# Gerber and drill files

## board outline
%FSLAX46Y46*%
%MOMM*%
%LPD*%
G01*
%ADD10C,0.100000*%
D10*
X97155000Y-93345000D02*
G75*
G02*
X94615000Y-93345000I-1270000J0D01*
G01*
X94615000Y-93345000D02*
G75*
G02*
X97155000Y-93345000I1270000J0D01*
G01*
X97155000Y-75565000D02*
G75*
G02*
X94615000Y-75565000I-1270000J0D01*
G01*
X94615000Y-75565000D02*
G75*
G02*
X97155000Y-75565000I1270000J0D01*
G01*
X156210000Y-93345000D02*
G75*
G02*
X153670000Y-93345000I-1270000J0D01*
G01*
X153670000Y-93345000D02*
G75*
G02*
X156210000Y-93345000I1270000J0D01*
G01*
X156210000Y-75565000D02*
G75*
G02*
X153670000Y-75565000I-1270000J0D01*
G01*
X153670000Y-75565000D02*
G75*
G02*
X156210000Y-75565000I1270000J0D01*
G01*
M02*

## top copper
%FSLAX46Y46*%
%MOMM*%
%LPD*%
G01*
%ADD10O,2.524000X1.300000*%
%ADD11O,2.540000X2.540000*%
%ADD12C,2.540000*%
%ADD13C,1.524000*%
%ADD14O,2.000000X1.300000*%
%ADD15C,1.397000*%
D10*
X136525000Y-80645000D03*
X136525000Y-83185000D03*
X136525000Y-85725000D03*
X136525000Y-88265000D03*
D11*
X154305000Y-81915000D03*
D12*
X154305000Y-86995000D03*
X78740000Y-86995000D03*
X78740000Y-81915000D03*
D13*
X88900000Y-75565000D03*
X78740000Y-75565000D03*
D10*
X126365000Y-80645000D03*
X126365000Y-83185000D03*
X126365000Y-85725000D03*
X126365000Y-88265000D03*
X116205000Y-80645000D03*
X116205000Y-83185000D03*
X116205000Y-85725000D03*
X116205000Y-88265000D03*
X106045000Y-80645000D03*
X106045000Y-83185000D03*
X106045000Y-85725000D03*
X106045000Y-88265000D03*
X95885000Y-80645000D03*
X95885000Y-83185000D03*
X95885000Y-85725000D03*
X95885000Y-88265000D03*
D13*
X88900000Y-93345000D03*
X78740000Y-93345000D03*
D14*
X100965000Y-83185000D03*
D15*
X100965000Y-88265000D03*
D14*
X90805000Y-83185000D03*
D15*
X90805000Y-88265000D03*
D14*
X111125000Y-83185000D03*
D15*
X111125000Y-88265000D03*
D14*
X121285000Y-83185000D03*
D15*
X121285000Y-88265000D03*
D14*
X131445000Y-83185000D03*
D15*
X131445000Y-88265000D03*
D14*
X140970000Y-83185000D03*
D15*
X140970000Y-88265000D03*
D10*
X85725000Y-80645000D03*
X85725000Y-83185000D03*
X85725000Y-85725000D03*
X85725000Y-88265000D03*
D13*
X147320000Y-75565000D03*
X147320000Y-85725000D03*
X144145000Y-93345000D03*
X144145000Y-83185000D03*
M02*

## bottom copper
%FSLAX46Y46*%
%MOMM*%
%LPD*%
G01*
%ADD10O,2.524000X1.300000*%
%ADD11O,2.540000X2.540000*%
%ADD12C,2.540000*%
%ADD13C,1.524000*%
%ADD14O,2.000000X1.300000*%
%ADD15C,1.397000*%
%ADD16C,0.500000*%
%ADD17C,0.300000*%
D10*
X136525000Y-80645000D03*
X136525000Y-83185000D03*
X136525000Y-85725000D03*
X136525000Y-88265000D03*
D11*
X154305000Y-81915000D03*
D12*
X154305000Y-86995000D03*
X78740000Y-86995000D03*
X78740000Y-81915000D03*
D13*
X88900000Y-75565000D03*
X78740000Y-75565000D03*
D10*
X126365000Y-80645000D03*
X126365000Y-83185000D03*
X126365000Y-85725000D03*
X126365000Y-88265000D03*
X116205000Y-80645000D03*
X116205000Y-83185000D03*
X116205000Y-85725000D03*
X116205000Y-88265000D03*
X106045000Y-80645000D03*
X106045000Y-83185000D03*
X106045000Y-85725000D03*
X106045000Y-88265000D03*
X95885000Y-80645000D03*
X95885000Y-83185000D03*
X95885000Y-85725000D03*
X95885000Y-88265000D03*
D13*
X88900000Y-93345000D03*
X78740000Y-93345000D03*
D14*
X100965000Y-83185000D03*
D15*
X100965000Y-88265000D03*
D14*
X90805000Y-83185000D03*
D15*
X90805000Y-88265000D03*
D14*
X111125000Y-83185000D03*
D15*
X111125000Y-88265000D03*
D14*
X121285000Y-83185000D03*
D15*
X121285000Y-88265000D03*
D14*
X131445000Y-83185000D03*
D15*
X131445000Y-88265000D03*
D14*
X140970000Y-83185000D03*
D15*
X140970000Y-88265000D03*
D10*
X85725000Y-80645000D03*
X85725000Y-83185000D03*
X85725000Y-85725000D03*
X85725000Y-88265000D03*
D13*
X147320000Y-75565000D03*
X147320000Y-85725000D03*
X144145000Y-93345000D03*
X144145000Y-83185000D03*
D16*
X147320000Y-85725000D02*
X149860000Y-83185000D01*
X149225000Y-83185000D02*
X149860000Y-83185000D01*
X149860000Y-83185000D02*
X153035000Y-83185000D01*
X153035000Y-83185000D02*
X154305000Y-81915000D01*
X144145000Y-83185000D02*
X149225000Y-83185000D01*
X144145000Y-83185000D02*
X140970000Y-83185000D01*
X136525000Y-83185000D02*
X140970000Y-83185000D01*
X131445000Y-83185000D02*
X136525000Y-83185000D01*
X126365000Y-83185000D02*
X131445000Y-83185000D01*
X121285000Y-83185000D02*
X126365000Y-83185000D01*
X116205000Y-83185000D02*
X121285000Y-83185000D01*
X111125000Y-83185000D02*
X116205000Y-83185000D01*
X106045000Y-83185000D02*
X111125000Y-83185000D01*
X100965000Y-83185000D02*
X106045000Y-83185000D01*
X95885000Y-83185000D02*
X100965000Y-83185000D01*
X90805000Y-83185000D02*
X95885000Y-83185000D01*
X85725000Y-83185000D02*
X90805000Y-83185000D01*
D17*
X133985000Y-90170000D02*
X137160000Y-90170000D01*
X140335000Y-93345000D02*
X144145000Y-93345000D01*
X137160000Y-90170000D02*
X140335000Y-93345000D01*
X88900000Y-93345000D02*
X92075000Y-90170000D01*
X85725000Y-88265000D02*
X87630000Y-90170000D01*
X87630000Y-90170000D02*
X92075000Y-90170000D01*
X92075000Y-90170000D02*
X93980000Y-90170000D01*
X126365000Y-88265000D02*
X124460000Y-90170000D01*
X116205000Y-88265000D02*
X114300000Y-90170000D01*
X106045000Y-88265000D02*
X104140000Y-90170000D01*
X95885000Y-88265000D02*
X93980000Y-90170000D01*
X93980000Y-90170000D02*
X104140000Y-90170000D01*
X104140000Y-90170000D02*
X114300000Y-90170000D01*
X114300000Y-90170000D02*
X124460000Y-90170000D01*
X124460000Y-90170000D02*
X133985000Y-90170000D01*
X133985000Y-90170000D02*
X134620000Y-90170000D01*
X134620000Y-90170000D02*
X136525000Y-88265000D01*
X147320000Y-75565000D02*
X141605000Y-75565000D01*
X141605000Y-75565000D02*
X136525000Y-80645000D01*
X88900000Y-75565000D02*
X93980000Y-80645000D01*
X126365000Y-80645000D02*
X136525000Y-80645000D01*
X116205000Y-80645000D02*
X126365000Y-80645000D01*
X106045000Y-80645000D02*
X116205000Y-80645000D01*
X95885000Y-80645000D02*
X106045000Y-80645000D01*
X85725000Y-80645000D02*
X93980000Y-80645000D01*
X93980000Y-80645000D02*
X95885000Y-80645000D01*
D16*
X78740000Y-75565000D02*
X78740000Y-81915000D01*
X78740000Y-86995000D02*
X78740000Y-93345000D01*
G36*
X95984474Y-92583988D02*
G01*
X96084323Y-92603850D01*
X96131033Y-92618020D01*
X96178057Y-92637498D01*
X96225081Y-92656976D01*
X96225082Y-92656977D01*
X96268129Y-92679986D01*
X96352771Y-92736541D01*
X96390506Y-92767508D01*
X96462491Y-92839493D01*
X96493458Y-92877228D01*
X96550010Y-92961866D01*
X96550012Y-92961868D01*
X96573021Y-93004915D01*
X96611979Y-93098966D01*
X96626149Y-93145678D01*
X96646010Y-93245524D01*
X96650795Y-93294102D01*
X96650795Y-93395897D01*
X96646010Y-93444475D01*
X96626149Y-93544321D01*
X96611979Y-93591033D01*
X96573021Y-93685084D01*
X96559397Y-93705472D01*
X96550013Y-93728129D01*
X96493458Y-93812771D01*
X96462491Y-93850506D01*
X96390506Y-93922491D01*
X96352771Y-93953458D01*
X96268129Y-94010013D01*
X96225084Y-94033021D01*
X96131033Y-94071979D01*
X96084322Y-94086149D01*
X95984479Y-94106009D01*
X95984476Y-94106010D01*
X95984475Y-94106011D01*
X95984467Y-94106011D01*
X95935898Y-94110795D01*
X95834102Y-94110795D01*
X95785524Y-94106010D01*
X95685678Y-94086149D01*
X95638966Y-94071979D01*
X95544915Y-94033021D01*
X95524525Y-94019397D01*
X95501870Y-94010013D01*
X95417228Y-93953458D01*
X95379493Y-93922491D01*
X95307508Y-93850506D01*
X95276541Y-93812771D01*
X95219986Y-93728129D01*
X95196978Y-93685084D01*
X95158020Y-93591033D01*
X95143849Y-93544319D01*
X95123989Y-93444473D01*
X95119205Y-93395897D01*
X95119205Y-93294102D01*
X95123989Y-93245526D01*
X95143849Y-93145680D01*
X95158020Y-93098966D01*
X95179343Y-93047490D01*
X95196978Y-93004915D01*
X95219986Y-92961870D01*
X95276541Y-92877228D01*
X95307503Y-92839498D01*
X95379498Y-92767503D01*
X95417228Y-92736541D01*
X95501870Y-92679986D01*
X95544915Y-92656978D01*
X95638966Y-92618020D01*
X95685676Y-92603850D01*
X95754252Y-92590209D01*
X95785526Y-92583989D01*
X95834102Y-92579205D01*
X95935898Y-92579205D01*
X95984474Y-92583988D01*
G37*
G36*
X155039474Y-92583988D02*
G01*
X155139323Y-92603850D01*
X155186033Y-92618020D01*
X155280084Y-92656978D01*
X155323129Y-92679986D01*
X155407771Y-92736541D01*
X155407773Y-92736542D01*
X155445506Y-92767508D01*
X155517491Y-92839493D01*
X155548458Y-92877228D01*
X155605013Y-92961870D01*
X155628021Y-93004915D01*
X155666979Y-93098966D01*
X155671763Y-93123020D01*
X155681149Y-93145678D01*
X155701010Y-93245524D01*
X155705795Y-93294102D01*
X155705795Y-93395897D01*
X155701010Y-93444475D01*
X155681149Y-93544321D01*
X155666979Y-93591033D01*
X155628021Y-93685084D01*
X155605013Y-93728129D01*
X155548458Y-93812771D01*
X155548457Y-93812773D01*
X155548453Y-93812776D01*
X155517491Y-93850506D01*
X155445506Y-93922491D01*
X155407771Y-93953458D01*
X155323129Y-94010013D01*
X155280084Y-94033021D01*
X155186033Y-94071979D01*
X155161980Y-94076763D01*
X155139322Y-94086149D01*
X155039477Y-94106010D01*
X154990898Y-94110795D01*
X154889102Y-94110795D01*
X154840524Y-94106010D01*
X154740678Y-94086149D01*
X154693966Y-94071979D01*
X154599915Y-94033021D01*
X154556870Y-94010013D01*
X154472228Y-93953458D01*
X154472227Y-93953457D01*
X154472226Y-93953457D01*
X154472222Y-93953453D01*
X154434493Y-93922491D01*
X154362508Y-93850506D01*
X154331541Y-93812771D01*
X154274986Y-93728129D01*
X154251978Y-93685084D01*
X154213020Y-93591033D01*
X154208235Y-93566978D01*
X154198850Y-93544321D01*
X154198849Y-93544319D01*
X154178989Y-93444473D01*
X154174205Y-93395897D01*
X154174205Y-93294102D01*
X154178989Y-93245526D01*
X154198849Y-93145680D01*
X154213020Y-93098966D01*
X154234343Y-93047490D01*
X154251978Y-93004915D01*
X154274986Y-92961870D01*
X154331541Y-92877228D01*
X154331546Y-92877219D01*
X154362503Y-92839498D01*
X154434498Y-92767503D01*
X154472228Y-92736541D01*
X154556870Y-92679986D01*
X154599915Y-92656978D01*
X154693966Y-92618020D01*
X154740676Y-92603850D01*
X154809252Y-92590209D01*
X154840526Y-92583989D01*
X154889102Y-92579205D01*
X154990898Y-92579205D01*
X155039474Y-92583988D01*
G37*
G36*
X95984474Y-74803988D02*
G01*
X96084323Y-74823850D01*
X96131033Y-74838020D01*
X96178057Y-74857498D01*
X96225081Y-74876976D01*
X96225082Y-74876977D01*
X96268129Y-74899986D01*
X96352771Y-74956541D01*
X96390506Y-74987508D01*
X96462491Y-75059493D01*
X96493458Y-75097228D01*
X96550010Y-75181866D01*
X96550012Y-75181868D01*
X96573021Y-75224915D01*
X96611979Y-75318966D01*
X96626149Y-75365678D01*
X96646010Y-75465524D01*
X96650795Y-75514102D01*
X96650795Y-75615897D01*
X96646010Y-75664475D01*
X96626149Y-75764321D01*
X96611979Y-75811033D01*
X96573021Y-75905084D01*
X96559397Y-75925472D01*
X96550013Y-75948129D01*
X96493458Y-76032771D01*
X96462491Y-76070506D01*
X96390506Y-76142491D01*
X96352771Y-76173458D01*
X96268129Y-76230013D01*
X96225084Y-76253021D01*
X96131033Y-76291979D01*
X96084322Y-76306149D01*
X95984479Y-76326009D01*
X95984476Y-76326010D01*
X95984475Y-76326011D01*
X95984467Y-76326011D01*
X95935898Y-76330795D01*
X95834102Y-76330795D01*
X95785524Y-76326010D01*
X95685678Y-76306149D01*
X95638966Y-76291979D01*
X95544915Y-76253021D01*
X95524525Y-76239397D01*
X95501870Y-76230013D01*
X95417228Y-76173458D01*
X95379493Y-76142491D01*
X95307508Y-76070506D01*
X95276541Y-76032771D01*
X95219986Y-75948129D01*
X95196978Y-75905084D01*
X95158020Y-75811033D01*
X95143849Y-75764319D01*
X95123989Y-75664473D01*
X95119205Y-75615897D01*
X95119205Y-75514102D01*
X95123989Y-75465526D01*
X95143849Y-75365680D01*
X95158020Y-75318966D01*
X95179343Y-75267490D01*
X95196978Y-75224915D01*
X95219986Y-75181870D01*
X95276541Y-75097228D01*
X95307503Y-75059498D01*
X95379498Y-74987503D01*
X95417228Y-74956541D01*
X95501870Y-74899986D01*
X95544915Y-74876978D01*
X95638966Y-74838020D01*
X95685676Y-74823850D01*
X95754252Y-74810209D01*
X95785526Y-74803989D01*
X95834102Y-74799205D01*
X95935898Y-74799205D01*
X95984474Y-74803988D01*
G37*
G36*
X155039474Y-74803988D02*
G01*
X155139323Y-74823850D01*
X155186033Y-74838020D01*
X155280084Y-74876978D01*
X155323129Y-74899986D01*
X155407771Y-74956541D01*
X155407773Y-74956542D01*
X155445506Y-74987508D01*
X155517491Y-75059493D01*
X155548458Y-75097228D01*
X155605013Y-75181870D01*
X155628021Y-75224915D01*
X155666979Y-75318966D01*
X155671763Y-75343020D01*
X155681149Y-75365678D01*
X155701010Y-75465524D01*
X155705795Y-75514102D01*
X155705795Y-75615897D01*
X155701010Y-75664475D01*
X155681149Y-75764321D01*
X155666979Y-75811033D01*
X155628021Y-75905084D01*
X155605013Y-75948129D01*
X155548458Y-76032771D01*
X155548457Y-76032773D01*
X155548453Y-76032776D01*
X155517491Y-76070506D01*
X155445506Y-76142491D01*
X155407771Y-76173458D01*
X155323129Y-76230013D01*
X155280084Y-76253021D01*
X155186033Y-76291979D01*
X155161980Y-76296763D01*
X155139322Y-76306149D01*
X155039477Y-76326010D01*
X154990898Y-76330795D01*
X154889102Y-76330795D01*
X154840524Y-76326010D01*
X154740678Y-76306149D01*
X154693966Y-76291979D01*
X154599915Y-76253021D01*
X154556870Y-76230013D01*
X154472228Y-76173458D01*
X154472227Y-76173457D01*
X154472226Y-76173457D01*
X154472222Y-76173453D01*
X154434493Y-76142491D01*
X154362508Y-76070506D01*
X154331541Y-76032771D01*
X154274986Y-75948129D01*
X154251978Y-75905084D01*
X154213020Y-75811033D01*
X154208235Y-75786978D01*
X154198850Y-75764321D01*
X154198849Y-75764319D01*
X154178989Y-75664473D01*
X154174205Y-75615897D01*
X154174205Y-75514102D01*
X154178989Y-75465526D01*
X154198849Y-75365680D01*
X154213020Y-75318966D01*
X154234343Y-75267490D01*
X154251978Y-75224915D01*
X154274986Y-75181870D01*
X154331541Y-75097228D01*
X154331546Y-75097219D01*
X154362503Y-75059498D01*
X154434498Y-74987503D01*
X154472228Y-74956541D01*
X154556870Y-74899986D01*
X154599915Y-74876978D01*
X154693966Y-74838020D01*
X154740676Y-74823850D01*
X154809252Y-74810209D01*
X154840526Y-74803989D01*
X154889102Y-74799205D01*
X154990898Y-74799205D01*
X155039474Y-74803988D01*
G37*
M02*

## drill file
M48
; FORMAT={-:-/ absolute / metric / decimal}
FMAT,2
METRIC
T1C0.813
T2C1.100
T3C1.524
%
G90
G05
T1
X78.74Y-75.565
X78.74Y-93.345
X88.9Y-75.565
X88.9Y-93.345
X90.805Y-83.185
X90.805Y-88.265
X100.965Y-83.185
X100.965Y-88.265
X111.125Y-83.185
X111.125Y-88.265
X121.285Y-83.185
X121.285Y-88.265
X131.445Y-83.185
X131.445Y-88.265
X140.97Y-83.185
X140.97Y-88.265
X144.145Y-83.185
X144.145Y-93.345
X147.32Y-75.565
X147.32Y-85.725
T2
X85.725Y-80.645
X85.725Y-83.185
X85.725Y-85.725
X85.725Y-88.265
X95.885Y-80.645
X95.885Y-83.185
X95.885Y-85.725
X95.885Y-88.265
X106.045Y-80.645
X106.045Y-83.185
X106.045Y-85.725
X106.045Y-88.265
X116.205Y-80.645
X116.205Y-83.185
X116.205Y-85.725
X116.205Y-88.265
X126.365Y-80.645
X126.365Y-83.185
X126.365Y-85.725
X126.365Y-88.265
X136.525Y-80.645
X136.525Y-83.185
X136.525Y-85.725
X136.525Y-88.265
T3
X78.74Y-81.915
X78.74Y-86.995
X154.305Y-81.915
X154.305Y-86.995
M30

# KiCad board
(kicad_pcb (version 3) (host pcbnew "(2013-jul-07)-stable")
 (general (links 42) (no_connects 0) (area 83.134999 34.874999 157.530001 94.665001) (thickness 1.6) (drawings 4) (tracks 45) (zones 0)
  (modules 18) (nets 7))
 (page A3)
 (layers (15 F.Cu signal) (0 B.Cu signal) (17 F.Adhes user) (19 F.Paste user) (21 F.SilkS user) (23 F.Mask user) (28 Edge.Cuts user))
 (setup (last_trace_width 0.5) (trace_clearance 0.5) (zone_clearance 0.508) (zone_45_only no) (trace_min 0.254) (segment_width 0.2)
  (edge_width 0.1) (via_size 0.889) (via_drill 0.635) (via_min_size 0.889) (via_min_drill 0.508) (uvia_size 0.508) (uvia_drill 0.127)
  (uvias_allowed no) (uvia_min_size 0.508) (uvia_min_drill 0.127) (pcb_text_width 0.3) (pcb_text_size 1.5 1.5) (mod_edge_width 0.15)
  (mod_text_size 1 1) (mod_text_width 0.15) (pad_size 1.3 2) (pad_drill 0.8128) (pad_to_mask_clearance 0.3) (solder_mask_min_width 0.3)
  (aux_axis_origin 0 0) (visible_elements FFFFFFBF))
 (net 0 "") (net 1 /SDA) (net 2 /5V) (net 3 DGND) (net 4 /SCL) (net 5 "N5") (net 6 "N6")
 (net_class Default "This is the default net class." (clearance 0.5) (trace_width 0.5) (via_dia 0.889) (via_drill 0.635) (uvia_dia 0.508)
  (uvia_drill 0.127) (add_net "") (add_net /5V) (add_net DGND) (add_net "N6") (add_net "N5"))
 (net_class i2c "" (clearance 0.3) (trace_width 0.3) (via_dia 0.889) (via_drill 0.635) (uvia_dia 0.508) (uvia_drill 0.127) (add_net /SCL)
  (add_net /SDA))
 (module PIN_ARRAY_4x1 (layer F.Cu) (at 136.525 84.455 270)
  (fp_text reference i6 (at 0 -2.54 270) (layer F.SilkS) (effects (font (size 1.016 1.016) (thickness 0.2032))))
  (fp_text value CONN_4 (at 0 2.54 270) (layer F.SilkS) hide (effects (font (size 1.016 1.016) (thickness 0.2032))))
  (pad 1 thru_hole oval (at -3.81 0 270) (size 1.3 2.524) (drill 1.1) (layers *.Cu *.Mask F.SilkS) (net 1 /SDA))
  (pad 2 thru_hole oval (at -1.27 0 270) (size 1.3 2.524) (drill 1.1) (layers *.Cu *.Mask F.SilkS) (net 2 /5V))
  (pad 3 thru_hole oval (at 1.27 0 270) (size 1.3 2.524) (drill 1.1) (layers *.Cu *.Mask F.SilkS) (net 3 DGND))
  (pad 4 thru_hole oval (at 3.81 0 270) (size 1.3 2.524) (drill 1.1) (layers *.Cu *.Mask F.SilkS) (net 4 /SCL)))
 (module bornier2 (layer F.Cu) (at 154.305 84.455 270)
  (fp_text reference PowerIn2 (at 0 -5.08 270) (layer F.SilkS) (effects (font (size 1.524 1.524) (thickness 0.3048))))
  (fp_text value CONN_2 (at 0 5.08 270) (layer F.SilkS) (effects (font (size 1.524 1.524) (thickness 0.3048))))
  (pad 1 thru_hole oval (at -2.54 0 270) (size 2.54 2.54) (drill 1.524) (layers *.Cu *.Mask F.SilkS) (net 2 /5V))
  (pad 2 thru_hole circle (at 2.54 0 270) (size 2.54 2.54) (drill 1.524) (layers *.Cu *.Mask F.SilkS) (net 3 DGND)))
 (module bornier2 (layer F.Cu) (at 78.74 84.455 90)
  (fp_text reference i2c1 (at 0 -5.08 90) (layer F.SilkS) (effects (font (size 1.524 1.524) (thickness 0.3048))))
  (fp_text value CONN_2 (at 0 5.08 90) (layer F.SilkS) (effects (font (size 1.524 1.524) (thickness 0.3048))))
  (pad 1 thru_hole circle (at -2.54 0 90) (size 2.54 2.54) (drill 1.524) (layers *.Cu *.Mask F.SilkS) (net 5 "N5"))
  (pad 2 thru_hole circle (at 2.54 0 90) (size 2.54 2.54) (drill 1.524) (layers *.Cu *.Mask F.SilkS) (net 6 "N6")))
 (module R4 (layer F.Cu) (at 83.82 75.565 180) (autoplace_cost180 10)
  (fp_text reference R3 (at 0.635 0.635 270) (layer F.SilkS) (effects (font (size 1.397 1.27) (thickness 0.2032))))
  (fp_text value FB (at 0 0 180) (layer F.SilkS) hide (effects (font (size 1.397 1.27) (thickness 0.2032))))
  (pad 1 thru_hole circle (at -5.08 0 180) (size 1.524 1.524) (drill 0.8128) (layers *.Cu *.Mask F.SilkS) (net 1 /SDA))
  (pad 2 thru_hole circle (at 5.08 0 180) (size 1.524 1.524) (drill 0.8128) (layers *.Cu *.Mask F.SilkS) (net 6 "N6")))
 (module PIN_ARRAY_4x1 (layer F.Cu) (at 126.365 84.455 270)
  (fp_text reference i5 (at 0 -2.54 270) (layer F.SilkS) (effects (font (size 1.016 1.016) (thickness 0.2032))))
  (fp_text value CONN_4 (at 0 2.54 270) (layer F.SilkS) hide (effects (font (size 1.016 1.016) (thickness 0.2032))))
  (pad 1 thru_hole oval (at -3.81 0 270) (size 1.3 2.524) (drill 1.1) (layers *.Cu *.Mask F.SilkS) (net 1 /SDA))
  (pad 2 thru_hole oval (at -1.27 0 270) (size 1.3 2.524) (drill 1.1) (layers *.Cu *.Mask F.SilkS) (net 2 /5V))
  (pad 3 thru_hole oval (at 1.27 0 270) (size 1.3 2.524) (drill 1.1) (layers *.Cu *.Mask F.SilkS) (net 3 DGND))
  (pad 4 thru_hole oval (at 3.81 0 270) (size 1.3 2.524) (drill 1.1) (layers *.Cu *.Mask F.SilkS) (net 4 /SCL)))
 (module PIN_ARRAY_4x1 (layer F.Cu) (at 116.205 84.455 270)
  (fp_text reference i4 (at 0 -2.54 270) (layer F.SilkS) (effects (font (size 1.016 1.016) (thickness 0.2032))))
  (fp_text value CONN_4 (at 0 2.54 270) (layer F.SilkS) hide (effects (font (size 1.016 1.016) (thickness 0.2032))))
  (pad 1 thru_hole oval (at -3.81 0 270) (size 1.3 2.524) (drill 1.1) (layers *.Cu *.Mask F.SilkS) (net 1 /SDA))
  (pad 2 thru_hole oval (at -1.27 0 270) (size 1.3 2.524) (drill 1.1) (layers *.Cu *.Mask F.SilkS) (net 2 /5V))
  (pad 3 thru_hole oval (at 1.27 0 270) (size 1.3 2.524) (drill 1.1) (layers *.Cu *.Mask F.SilkS) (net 3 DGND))
  (pad 4 thru_hole oval (at 3.81 0 270) (size 1.3 2.524) (drill 1.1) (layers *.Cu *.Mask F.SilkS) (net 4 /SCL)))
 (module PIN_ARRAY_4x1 (layer F.Cu) (at 106.045 84.455 270)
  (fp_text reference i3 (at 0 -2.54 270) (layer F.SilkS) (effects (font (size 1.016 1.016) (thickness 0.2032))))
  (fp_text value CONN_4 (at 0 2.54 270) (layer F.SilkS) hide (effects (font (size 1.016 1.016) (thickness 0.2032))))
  (pad 1 thru_hole oval (at -3.81 0 270) (size 1.3 2.524) (drill 1.1) (layers *.Cu *.Mask F.SilkS) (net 1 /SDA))
  (pad 2 thru_hole oval (at -1.27 0 270) (size 1.3 2.524) (drill 1.1) (layers *.Cu *.Mask F.SilkS) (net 2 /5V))
  (pad 3 thru_hole oval (at 1.27 0 270) (size 1.3 2.524) (drill 1.1) (layers *.Cu *.Mask F.SilkS) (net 3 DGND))
  (pad 4 thru_hole oval (at 3.81 0 270) (size 1.3 2.524) (drill 1.1) (layers *.Cu *.Mask F.SilkS) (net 4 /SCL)))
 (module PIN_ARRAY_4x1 (layer F.Cu) (at 95.885 84.455 270)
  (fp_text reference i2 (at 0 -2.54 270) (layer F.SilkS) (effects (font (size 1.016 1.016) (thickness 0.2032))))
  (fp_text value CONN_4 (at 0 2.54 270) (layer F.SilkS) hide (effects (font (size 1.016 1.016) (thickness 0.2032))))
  (pad 1 thru_hole oval (at -3.81 0 270) (size 1.3 2.524) (drill 1.1) (layers *.Cu *.Mask F.SilkS) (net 1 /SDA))
  (pad 2 thru_hole oval (at -1.27 0 270) (size 1.3 2.524) (drill 1.1) (layers *.Cu *.Mask F.SilkS) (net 2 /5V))
  (pad 3 thru_hole oval (at 1.27 0 270) (size 1.3 2.524) (drill 1.1) (layers *.Cu *.Mask F.SilkS) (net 3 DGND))
  (pad 4 thru_hole oval (at 3.81 0 270) (size 1.3 2.524) (drill 1.1) (layers *.Cu *.Mask F.SilkS) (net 4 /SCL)))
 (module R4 (layer F.Cu) (at 83.82 93.345 180) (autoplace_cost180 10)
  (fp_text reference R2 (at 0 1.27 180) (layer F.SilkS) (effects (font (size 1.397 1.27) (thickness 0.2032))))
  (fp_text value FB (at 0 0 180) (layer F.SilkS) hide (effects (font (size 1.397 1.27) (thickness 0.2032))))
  (pad 1 thru_hole circle (at -5.08 0 180) (size 1.524 1.524) (drill 0.8128) (layers *.Cu *.Mask F.SilkS) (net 4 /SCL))
  (pad 2 thru_hole circle (at 5.08 0 180) (size 1.524 1.524) (drill 0.8128) (layers *.Cu *.Mask F.SilkS) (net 5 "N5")))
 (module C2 (layer F.Cu) (at 100.965 85.725 270)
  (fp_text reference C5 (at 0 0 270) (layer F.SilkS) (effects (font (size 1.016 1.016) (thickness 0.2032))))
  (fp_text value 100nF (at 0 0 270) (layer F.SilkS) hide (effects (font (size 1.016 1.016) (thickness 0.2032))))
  (pad 1 thru_hole oval (at -2.54 0 270) (size 1.3 2) (drill 0.8128) (layers *.Cu *.Mask F.SilkS) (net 2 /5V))
  (pad 2 thru_hole circle (at 2.54 0 270) (size 1.397 1.397) (drill 0.8128) (layers *.Cu *.Mask F.SilkS) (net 3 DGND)))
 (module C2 (layer F.Cu) (at 90.805 85.725 270)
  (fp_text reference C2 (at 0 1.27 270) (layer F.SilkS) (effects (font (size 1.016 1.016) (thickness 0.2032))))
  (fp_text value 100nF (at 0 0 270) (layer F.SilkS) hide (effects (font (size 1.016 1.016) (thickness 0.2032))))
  (pad 1 thru_hole oval (at -2.54 0 270) (size 1.3 2) (drill 0.8128) (layers *.Cu *.Mask F.SilkS) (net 2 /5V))
  (pad 2 thru_hole circle (at 2.54 0 270) (size 1.397 1.397) (drill 0.8128) (layers *.Cu *.Mask F.SilkS) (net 3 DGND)))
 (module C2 (layer F.Cu) (at 111.125 85.725 270)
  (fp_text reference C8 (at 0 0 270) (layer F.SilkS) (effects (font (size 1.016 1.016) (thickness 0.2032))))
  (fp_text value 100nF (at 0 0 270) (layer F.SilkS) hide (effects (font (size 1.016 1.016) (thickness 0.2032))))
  (pad 1 thru_hole oval (at -2.54 0 270) (size 1.3 2) (drill 0.8128) (layers *.Cu *.Mask F.SilkS) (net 2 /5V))
  (pad 2 thru_hole circle (at 2.54 0 270) (size 1.397 1.397) (drill 0.8128) (layers *.Cu *.Mask F.SilkS) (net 3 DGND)))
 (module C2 (layer F.Cu) (at 121.285 85.725 270)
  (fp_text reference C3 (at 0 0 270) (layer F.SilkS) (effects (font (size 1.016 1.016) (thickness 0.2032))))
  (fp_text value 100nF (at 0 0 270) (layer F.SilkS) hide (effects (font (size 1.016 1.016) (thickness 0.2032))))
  (pad 1 thru_hole oval (at -2.54 0 270) (size 1.3 2) (drill 0.8128) (layers *.Cu *.Mask F.SilkS) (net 2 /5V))
  (pad 2 thru_hole circle (at 2.54 0 270) (size 1.397 1.397) (drill 0.8128) (layers *.Cu *.Mask F.SilkS) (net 3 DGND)))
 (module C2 (layer F.Cu) (at 131.445 85.725 270)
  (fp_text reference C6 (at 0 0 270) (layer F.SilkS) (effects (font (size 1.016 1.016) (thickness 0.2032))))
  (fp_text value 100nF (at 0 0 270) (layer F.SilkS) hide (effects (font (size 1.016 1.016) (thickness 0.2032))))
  (pad 1 thru_hole oval (at -2.54 0 270) (size 1.3 2) (drill 0.8128) (layers *.Cu *.Mask F.SilkS) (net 2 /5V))
  (pad 2 thru_hole circle (at 2.54 0 270) (size 1.397 1.397) (drill 0.8128) (layers *.Cu *.Mask F.SilkS) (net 3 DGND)))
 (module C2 (layer F.Cu) (at 140.97 85.725 270)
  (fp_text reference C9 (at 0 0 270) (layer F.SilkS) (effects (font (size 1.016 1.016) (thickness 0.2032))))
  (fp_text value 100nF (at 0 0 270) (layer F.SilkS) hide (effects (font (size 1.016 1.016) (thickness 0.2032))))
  (pad 1 thru_hole oval (at -2.54 0 270) (size 1.3 2) (drill 0.8128) (layers *.Cu *.Mask F.SilkS) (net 2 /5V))
  (pad 2 thru_hole circle (at 2.54 0 270) (size 1.397 1.397) (drill 0.8128) (layers *.Cu *.Mask F.SilkS) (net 3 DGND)))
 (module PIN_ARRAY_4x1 (layer F.Cu) (at 85.725 84.455 90)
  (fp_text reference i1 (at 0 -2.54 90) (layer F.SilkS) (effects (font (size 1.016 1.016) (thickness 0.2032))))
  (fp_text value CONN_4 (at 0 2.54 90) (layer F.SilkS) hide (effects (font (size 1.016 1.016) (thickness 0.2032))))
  (pad 1 thru_hole oval (at 3.81 0 90) (size 1.3 2.524) (drill 1.1) (layers *.Cu *.Mask F.SilkS) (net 1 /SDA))
  (pad 2 thru_hole oval (at 1.27 0 90) (size 1.3 2.524) (drill 1.1) (layers *.Cu *.Mask F.SilkS) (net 2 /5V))
  (pad 3 thru_hole oval (at -1.27 0 90) (size 1.3 2.524) (drill 1.1) (layers *.Cu *.Mask F.SilkS) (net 3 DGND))
  (pad 4 thru_hole oval (at -3.81 0 90) (size 1.3 2.524) (drill 1.1) (layers *.Cu *.Mask F.SilkS) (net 4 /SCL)))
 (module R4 (layer F.Cu) (at 147.32 80.645 270) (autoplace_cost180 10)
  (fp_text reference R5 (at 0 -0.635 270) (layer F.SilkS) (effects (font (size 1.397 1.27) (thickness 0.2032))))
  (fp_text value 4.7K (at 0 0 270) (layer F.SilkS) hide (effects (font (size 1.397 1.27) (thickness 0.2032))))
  (pad 1 thru_hole circle (at -5.08 0 270) (size 1.524 1.524) (drill 0.8128) (layers *.Cu *.Mask F.SilkS) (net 1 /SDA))
  (pad 2 thru_hole circle (at 5.08 0 270) (size 1.524 1.524) (drill 0.8128) (layers *.Cu *.Mask F.SilkS) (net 2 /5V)))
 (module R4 (layer F.Cu) (at 144.145 88.265 90) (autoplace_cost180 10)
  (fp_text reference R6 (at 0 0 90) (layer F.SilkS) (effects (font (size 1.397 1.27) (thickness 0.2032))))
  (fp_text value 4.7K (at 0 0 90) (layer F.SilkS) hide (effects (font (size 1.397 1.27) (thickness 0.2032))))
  (pad 1 thru_hole circle (at -5.08 0 90) (size 1.524 1.524) (drill 0.8128) (layers *.Cu *.Mask F.SilkS) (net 4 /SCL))
  (pad 2 thru_hole circle (at 5.08 0 90) (size 1.524 1.524) (drill 0.8128) (layers *.Cu *.Mask F.SilkS) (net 2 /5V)))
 (gr_circle (center 95.885 93.345) (end 97.155 93.345) (layer Edge.Cuts) (width 0.1))
 (gr_circle (center 95.885 75.565) (end 97.155 75.565) (layer Edge.Cuts) (width 0.1))
 (gr_circle (center 154.94 93.345) (end 156.21 93.345) (layer Edge.Cuts) (width 0.1))
 (gr_circle (center 154.94 75.565) (end 153.67 75.565) (layer Edge.Cuts) (width 0.1))
 (segment (start 147.32 85.725) (end 149.86 83.185) (width 0.5) (layer B.Cu) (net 2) (status 400000))
 (segment (start 149.225 83.185) (end 149.86 83.185) (width 0.5) (layer B.Cu) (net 2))
 (segment (start 149.86 83.185) (end 153.035 83.185) (width 0.5) (layer B.Cu) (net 2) (status 800000))
 (segment (start 153.035 83.185) (end 154.305 81.915) (width 0.5) (layer B.Cu) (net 2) (status C00000))
 (segment (start 144.145 83.185) (end 149.225 83.185) (width 0.5) (layer B.Cu) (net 2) (status 400000))
 (segment (start 144.145 83.185) (end 140.97 83.185) (width 0.5) (layer B.Cu) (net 2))
 (segment (start 136.525 83.185) (end 140.97 83.185) (width 0.5) (layer B.Cu) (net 2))
 (segment (start 131.445 83.185) (end 136.525 83.185) (width 0.5) (layer B.Cu) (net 2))
 (segment (start 126.365 83.185) (end 131.445 83.185) (width 0.5) (layer B.Cu) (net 2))
 (segment (start 121.285 83.185) (end 126.365 83.185) (width 0.5) (layer B.Cu) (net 2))
 (segment (start 116.205 83.185) (end 121.285 83.185) (width 0.5) (layer B.Cu) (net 2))
 (segment (start 111.125 83.185) (end 116.205 83.185) (width 0.5) (layer B.Cu) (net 2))
 (segment (start 106.045 83.185) (end 111.125 83.185) (width 0.5) (layer B.Cu) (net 2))
 (segment (start 100.965 83.185) (end 106.045 83.185) (width 0.5) (layer B.Cu) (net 2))
 (segment (start 95.885 83.185) (end 100.965 83.185) (width 0.5) (layer B.Cu) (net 2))
 (segment (start 90.805 83.185) (end 95.885 83.185) (width 0.5) (layer B.Cu) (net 2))
 (segment (start 85.725 83.185) (end 90.805 83.185) (width 0.5) (layer B.Cu) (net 2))
 (segment (start 133.985 90.17) (end 137.16 90.17) (width 0.3) (layer B.Cu) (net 4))
 (segment (start 140.335 93.345) (end 144.145 93.345) (width 0.3) (layer B.Cu) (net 4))
 (segment (start 137.16 90.17) (end 140.335 93.345) (width 0.3) (layer B.Cu) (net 4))
 (segment (start 88.9 93.345) (end 92.075 90.17) (width 0.3) (layer B.Cu) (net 4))
 (segment (start 85.725 88.265) (end 87.63 90.17) (width 0.3) (layer B.Cu) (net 4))
 (segment (start 87.63 90.17) (end 92.075 90.17) (width 0.3) (layer B.Cu) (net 4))
 (segment (start 92.075 90.17) (end 93.98 90.17) (width 0.3) (layer B.Cu) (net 4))
 (segment (start 126.365 88.265) (end 124.46 90.17) (width 0.3) (layer B.Cu) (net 4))
 (segment (start 116.205 88.265) (end 114.3 90.17) (width 0.3) (layer B.Cu) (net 4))
 (segment (start 106.045 88.265) (end 104.14 90.17) (width 0.3) (layer B.Cu) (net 4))
 (segment (start 95.885 88.265) (end 93.98 90.17) (width 0.3) (layer B.Cu) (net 4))
 (segment (start 93.98 90.17) (end 104.14 90.17) (width 0.3) (layer B.Cu) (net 4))
 (segment (start 104.14 90.17) (end 114.3 90.17) (width 0.3) (layer B.Cu) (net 4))
 (segment (start 114.3 90.17) (end 124.46 90.17) (width 0.3) (layer B.Cu) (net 4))
 (segment (start 124.46 90.17) (end 133.985 90.17) (width 0.3) (layer B.Cu) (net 4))
 (segment (start 133.985 90.17) (end 134.62 90.17) (width 0.3) (layer B.Cu) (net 4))
 (segment (start 134.62 90.17) (end 136.525 88.265) (width 0.3) (layer B.Cu) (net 4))
 (segment (start 147.32 75.565) (end 141.605 75.565) (width 0.3) (layer B.Cu) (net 1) (status 400000))
 (segment (start 141.605 75.565) (end 136.525 80.645) (width 0.3) (layer B.Cu) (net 1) (status 800000))
 (segment (start 88.9 75.565) (end 93.98 80.645) (width 0.3) (layer B.Cu) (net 1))
 (segment (start 126.365 80.645) (end 136.525 80.645) (width 0.3) (layer B.Cu) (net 1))
 (segment (start 116.205 80.645) (end 126.365 80.645) (width 0.3) (layer B.Cu) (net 1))
 (segment (start 106.045 80.645) (end 116.205 80.645) (width 0.3) (layer B.Cu) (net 1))
 (segment (start 95.885 80.645) (end 106.045 80.645) (width 0.3) (layer B.Cu) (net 1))
 (segment (start 85.725 80.645) (end 93.98 80.645) (width 0.3) (layer B.Cu) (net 1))
 (segment (start 93.98 80.645) (end 95.885 80.645) (width 0.3) (layer B.Cu) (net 1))
 (segment (start 78.74 75.565) (end 78.74 81.915) (width 0.5) (layer B.Cu) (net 6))
 (segment (start 78.74 86.995) (end 78.74 93.345) (width 0.5) (layer B.Cu) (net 5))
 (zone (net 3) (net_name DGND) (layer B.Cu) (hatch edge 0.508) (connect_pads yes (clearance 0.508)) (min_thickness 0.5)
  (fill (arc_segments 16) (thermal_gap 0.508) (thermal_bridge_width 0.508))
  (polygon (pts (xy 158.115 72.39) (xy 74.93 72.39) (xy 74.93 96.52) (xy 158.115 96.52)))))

